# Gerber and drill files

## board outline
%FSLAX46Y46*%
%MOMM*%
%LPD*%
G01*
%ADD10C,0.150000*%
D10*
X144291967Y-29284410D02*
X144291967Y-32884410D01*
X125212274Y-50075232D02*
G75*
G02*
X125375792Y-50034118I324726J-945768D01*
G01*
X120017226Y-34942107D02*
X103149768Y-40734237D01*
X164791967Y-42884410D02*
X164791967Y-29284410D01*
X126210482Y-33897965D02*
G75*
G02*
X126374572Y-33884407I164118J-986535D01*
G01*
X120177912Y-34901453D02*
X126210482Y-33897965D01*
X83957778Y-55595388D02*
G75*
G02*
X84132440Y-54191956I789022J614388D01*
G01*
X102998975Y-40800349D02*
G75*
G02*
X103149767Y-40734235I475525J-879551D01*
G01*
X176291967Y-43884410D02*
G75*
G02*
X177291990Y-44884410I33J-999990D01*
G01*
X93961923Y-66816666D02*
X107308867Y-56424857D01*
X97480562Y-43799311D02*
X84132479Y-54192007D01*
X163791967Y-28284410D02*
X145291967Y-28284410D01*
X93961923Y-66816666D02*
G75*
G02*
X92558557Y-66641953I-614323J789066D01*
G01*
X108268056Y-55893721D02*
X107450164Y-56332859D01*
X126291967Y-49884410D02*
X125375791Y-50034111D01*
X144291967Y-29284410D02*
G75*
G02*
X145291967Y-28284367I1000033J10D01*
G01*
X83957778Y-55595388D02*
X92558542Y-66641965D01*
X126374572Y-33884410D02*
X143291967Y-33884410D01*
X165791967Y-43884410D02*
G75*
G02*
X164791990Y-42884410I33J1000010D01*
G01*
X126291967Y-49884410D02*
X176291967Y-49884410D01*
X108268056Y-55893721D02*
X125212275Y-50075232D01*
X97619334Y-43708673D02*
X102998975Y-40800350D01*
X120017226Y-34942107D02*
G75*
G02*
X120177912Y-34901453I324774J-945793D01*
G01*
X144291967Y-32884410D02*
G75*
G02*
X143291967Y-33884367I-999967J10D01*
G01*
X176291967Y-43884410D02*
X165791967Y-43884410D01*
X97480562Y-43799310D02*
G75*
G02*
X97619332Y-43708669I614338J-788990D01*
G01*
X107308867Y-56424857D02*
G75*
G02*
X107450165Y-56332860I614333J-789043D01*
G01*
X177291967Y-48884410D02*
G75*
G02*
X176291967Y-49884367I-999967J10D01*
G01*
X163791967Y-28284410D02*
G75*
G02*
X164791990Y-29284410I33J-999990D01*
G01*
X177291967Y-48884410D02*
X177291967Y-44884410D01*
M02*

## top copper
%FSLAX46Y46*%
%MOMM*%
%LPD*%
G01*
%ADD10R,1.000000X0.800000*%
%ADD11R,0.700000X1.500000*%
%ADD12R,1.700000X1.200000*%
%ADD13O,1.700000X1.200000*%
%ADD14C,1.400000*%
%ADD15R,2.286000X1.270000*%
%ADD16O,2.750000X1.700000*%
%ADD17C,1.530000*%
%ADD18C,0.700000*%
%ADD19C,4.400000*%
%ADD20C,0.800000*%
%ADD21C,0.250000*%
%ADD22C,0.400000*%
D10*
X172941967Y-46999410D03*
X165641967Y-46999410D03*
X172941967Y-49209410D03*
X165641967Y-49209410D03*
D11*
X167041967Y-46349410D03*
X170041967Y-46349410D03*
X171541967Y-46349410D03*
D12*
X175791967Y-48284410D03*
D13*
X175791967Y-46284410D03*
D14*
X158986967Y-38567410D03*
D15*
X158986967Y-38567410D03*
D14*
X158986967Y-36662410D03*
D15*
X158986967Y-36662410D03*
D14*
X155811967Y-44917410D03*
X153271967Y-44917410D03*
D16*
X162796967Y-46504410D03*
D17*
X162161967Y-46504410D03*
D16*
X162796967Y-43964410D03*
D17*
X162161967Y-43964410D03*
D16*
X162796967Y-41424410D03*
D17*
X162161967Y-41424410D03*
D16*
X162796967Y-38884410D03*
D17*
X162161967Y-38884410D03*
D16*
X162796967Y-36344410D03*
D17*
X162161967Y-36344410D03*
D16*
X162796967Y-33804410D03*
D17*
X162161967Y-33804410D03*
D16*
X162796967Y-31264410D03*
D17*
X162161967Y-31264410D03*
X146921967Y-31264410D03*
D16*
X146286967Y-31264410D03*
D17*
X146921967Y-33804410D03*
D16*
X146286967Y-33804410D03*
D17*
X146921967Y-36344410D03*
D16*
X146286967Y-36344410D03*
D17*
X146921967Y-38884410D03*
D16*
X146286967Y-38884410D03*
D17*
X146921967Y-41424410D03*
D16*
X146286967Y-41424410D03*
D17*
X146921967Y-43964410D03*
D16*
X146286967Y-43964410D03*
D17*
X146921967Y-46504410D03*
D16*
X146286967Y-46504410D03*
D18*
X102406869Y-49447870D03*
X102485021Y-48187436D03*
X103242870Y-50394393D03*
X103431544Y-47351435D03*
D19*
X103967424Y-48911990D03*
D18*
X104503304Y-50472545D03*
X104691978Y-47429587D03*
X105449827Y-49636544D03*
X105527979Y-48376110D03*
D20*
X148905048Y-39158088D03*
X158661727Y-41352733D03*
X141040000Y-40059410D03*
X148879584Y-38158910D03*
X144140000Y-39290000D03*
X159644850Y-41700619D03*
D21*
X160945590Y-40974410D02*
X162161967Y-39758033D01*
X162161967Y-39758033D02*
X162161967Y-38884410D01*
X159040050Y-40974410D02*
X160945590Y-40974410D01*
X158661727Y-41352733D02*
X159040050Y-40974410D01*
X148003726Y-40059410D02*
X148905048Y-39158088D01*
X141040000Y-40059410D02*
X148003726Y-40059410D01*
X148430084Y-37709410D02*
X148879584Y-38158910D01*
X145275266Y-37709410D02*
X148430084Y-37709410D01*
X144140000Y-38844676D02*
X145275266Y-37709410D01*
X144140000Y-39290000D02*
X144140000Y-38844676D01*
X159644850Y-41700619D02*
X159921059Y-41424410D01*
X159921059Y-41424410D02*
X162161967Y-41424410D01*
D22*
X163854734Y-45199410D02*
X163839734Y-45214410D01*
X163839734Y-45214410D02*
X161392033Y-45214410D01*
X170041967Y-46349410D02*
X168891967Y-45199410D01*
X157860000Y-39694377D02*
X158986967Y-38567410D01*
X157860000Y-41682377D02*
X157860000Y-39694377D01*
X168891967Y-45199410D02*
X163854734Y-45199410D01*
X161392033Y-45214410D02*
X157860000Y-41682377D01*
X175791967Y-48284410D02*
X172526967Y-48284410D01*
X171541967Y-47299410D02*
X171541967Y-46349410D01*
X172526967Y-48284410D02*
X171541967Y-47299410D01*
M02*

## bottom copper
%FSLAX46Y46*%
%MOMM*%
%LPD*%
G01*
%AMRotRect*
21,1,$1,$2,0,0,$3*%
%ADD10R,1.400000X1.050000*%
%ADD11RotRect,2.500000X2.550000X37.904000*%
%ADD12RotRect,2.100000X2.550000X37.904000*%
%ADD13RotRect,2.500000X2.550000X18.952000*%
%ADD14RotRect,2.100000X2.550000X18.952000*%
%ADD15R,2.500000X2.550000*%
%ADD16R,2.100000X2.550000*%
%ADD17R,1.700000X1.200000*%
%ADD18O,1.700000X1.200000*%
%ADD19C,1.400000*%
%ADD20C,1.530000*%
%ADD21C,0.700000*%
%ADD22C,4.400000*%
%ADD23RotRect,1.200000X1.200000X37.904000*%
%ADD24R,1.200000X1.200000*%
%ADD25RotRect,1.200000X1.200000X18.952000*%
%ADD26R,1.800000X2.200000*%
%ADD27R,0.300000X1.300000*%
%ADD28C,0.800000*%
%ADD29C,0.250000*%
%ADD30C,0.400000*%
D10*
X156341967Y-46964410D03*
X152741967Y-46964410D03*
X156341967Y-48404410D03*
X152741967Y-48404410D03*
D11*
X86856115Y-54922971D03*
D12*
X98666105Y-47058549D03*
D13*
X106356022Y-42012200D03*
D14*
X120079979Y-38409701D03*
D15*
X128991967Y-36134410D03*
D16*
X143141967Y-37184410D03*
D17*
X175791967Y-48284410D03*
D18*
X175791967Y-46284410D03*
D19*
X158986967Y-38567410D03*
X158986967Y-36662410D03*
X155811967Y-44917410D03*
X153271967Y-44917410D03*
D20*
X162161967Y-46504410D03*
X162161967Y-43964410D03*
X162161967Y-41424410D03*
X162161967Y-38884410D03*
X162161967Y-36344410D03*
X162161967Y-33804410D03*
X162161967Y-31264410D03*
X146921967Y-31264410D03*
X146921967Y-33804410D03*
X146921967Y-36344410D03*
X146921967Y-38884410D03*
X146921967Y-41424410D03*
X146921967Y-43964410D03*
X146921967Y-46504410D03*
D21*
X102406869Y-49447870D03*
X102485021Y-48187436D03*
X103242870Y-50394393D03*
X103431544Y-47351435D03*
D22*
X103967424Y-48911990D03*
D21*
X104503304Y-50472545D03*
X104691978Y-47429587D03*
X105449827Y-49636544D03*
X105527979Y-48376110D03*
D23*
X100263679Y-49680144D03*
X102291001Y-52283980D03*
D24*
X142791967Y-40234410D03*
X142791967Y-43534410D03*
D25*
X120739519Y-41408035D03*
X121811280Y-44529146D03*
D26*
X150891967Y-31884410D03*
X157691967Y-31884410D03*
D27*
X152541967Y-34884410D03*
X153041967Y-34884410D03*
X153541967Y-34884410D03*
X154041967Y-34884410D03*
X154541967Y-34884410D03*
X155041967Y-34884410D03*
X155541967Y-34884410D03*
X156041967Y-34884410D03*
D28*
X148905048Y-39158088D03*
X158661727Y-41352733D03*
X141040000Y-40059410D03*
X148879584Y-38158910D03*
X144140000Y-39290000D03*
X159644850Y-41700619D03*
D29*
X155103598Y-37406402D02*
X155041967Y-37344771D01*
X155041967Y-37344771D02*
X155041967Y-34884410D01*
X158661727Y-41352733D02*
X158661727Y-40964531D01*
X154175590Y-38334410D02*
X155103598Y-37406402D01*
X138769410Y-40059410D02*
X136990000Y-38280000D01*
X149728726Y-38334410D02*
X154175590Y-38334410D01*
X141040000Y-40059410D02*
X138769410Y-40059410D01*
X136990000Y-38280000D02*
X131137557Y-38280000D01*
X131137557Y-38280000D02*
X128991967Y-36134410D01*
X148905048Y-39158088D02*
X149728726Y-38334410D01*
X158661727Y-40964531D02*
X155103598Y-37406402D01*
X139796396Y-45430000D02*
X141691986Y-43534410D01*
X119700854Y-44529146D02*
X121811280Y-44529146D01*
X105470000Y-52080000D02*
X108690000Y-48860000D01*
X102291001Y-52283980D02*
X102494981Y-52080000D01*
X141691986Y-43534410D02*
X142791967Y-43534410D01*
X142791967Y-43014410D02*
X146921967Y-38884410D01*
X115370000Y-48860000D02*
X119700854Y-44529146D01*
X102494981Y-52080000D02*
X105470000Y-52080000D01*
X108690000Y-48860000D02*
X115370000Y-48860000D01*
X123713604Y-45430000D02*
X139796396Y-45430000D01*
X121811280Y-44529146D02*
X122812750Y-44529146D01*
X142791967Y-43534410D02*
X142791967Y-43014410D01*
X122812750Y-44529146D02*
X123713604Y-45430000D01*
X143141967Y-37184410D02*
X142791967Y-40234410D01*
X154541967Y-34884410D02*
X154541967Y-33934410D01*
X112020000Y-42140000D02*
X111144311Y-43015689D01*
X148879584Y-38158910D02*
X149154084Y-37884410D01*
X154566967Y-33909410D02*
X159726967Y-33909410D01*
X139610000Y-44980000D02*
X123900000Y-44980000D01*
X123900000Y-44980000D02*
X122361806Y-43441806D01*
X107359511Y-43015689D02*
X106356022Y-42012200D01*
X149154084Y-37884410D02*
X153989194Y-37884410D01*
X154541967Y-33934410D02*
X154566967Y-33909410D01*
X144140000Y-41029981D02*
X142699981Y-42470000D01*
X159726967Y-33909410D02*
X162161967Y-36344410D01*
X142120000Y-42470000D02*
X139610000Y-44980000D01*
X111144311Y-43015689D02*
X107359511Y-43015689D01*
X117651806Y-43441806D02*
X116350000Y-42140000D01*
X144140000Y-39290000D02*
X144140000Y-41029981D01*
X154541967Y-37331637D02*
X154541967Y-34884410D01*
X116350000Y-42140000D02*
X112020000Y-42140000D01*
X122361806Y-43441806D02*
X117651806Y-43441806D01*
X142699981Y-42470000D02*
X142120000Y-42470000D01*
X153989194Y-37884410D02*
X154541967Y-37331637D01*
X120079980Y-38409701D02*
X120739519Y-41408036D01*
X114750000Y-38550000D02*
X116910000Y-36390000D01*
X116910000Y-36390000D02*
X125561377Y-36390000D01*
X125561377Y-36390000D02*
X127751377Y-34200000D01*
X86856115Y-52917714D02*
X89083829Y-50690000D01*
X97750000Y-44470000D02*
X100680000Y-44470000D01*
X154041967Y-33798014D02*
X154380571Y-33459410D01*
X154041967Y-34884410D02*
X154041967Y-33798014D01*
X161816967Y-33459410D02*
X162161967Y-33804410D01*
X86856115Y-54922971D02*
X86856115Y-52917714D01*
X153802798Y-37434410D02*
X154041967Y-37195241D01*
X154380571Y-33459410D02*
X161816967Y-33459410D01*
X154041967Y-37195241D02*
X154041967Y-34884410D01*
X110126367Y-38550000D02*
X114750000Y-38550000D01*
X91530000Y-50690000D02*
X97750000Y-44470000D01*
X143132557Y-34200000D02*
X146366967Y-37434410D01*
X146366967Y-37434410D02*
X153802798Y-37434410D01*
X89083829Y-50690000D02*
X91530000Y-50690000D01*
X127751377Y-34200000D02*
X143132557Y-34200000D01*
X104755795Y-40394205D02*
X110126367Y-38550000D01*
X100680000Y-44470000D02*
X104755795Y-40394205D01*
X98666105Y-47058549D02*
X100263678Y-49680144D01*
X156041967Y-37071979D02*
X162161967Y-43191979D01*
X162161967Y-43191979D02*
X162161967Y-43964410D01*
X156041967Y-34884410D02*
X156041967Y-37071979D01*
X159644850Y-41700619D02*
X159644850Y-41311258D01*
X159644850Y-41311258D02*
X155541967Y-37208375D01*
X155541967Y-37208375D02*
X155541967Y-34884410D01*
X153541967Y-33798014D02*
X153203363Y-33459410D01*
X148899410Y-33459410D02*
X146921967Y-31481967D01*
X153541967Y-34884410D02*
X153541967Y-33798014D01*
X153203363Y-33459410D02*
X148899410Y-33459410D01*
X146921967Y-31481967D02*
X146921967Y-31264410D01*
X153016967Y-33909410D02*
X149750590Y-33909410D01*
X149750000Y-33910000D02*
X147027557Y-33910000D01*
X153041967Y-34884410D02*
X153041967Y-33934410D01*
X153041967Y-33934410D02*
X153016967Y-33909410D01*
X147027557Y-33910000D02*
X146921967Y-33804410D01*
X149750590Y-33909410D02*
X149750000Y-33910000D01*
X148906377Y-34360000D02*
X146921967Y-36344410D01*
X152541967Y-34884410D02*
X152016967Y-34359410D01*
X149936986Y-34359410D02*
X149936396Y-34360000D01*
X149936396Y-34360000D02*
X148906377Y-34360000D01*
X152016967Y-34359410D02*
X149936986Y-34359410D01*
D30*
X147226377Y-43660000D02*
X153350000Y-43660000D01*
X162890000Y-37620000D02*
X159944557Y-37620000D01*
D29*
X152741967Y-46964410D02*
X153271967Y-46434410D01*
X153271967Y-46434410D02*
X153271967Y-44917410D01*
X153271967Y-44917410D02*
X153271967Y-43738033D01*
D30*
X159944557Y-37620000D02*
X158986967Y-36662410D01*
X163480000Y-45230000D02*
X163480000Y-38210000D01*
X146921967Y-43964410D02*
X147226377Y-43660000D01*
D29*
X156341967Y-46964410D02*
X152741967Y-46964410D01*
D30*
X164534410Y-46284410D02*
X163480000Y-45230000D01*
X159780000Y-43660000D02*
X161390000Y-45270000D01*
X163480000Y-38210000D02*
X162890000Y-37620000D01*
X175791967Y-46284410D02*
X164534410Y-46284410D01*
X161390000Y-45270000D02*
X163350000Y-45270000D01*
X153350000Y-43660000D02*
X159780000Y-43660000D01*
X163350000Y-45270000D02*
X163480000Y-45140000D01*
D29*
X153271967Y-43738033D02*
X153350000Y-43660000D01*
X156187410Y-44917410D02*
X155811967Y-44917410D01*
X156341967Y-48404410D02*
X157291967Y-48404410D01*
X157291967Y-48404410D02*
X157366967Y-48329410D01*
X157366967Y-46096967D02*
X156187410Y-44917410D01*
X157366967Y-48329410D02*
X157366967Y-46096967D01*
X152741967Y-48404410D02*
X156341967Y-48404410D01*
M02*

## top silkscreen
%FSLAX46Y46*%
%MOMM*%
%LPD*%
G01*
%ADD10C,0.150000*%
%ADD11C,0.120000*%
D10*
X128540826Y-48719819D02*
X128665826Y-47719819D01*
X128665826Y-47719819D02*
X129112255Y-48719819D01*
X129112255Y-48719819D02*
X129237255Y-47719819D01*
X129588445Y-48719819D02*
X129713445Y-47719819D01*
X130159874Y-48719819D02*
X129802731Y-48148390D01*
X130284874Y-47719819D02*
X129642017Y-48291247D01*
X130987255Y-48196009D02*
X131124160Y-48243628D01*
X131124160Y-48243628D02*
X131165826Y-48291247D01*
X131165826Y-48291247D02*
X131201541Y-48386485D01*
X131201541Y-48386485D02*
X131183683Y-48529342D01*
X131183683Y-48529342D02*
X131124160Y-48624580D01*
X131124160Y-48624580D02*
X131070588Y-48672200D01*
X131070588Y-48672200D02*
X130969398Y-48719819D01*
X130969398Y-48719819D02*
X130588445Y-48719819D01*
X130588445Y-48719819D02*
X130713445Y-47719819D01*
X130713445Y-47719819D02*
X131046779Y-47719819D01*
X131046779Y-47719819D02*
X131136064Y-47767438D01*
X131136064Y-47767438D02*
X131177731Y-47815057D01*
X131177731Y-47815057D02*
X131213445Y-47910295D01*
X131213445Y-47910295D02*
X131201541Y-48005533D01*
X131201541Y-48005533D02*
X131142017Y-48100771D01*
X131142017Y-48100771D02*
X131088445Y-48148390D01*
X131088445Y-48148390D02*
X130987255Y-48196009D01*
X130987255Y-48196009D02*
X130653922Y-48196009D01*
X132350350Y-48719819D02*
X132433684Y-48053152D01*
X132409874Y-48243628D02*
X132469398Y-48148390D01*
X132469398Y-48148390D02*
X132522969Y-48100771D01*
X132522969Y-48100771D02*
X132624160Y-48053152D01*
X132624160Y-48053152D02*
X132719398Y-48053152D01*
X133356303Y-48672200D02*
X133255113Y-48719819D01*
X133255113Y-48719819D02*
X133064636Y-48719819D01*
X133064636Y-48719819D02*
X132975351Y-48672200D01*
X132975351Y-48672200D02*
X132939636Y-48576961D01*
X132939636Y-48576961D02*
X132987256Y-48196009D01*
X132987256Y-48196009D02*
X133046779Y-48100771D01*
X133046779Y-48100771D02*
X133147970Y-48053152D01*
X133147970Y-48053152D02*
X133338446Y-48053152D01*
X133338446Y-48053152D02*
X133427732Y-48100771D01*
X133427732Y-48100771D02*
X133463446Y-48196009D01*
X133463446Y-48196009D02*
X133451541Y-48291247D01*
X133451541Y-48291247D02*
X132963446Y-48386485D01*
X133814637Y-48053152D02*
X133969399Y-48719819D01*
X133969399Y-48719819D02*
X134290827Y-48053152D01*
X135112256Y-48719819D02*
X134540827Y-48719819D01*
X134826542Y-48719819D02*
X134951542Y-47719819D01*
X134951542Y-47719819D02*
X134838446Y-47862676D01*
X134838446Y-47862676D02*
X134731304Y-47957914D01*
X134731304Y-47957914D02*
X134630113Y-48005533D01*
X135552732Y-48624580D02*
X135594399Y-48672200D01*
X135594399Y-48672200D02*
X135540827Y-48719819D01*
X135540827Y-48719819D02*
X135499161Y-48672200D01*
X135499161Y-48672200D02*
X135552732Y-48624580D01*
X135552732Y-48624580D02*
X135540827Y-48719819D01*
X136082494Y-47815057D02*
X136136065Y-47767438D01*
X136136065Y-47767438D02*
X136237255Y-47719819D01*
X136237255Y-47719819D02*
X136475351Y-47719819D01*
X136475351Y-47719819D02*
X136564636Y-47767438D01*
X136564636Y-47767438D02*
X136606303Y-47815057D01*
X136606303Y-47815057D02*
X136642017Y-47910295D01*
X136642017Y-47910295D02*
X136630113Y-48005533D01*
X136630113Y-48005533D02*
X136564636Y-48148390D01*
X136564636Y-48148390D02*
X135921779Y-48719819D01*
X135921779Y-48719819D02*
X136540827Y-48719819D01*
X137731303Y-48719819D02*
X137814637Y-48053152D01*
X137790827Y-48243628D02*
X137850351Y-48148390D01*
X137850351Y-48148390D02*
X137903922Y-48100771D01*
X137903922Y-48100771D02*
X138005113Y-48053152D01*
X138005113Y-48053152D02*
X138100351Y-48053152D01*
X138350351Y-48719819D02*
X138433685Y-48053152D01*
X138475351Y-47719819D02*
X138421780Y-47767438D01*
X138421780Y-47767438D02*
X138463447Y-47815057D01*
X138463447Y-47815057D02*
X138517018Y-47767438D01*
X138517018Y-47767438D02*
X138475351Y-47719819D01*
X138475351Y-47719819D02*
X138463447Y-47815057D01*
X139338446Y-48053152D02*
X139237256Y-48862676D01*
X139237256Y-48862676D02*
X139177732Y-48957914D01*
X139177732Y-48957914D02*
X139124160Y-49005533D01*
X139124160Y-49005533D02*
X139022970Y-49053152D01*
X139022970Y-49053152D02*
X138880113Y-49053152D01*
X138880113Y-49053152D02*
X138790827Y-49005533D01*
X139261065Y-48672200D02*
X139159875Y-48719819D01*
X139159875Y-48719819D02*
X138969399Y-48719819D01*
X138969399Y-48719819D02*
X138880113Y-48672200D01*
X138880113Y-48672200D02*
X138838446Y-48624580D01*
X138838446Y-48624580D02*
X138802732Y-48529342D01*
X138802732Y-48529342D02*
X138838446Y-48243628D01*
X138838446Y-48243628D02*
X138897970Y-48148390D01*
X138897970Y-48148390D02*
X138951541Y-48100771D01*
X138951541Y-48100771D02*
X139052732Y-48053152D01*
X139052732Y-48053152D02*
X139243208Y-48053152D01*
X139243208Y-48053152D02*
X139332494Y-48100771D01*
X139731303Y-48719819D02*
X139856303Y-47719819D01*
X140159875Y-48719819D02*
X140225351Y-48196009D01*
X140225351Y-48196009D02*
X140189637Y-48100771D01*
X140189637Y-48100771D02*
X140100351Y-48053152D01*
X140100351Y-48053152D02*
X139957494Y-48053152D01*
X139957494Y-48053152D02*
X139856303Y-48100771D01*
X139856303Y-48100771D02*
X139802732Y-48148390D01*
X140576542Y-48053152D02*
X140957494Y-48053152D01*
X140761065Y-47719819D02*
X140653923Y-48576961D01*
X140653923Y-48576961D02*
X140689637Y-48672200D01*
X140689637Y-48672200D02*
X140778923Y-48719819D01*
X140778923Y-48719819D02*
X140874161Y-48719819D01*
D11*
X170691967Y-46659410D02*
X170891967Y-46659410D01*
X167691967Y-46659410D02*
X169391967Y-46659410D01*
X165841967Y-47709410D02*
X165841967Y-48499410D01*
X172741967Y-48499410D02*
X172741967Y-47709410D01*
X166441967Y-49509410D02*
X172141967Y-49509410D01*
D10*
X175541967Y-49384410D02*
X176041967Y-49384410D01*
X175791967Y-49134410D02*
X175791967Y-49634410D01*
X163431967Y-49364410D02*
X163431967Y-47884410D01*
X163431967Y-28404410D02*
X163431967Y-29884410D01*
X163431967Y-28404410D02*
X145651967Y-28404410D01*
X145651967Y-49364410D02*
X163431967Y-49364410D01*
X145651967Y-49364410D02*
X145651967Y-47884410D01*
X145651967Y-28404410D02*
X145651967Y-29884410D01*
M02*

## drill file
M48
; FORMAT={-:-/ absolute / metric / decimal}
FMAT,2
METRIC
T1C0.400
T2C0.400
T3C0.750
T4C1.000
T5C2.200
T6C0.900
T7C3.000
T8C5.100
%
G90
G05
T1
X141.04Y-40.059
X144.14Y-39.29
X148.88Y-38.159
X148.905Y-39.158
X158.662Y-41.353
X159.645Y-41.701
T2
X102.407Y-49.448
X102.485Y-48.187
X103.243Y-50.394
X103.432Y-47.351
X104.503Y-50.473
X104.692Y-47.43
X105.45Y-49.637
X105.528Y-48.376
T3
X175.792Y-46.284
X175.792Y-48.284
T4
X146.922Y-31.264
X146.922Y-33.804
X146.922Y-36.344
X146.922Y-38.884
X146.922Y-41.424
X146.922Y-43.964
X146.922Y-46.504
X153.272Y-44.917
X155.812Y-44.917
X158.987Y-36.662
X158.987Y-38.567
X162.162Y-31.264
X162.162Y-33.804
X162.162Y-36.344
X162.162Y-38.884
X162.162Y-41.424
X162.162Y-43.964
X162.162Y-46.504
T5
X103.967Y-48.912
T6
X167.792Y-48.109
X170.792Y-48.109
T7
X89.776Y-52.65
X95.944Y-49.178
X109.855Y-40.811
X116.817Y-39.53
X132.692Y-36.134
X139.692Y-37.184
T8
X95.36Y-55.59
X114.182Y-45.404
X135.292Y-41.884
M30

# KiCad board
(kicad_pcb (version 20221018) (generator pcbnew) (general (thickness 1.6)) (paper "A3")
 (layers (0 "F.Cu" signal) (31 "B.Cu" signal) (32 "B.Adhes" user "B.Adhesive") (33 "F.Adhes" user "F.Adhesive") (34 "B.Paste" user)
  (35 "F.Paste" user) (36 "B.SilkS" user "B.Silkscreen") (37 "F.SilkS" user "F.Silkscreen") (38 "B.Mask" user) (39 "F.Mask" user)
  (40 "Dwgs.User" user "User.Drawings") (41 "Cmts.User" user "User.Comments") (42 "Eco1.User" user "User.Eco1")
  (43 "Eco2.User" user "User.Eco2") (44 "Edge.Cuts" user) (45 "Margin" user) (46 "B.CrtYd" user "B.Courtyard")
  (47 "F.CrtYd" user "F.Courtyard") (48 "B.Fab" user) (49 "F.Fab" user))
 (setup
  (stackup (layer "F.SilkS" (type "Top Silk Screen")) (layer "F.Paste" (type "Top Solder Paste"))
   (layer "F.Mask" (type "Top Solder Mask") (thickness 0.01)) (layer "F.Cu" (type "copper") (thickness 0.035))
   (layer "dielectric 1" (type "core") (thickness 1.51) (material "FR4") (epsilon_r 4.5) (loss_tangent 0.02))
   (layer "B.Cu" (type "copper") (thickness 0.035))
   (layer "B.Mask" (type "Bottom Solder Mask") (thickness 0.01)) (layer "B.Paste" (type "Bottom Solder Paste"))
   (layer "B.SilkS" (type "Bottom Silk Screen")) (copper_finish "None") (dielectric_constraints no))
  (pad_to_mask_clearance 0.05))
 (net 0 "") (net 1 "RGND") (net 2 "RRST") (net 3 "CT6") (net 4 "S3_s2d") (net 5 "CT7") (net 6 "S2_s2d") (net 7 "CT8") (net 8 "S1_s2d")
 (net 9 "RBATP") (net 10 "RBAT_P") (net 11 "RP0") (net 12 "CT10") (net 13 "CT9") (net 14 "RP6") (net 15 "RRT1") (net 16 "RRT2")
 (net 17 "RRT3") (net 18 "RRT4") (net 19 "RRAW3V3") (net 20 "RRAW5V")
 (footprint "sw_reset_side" (layer "F.Cu") (at 154.541967 47.68441 -90)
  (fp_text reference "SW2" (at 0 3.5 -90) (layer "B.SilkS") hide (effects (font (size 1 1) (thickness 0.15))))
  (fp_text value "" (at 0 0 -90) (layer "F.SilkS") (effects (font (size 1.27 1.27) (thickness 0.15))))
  (pad "1" smd rect (at -0.72 -1.8 180) (size 1.4 1.05) (layers "B.Cu" "B.Paste" "B.Mask") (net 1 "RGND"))
  (pad "1" smd rect (at -0.72 1.8 180) (size 1.4 1.05) (layers "B.Cu" "B.Paste" "B.Mask") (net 1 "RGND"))
  (pad "2" smd rect (at 0.72 -1.8 180) (size 1.4 1.05) (layers "B.Cu" "B.Paste" "B.Mask") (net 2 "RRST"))
  (pad "2" smd rect (at 0.72 1.8 180) (size 1.4 1.05) (layers "B.Cu" "B.Paste" "B.Mask") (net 2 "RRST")))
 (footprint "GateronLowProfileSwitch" (layer "F.Cu") (at 95.359531 55.589614 37.904)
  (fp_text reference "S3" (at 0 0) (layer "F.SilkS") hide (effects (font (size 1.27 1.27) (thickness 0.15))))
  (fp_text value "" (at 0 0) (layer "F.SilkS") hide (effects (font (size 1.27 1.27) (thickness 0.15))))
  (pad "" np_thru_hole circle (at -2.6 -5.75) (size 3 3) (drill 3) (layers "*.Cu" "*.Mask"))
  (pad "" np_thru_hole circle (at 0 0) (size 5.1 5.1) (drill 5.1) (layers "*.Cu" "*.Mask"))
  (pad "" np_thru_hole circle (at 4.4 -4.7) (size 3 3) (drill 3) (layers "*.Cu" "*.Mask"))
  (pad "1" smd rect (at -6.3 -5.75 37.904) (size 2.5 2.55) (layers "B.Cu" "B.Paste" "B.Mask") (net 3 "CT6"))
  (pad "2" smd rect (at 7.85 -4.7 37.904) (size 2.1 2.55) (layers "B.Cu" "B.Paste" "B.Mask") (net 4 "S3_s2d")))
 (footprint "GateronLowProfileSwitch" (layer "F.Cu") (at 114.181967 45.40441 18.952)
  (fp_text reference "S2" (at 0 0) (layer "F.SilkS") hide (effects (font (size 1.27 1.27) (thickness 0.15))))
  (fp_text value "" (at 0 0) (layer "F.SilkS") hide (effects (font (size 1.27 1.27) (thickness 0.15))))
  (pad "" np_thru_hole circle (at -2.6 -5.75) (size 3 3) (drill 3) (layers "*.Cu" "*.Mask"))
  (pad "" np_thru_hole circle (at 0 0) (size 5.1 5.1) (drill 5.1) (layers "*.Cu" "*.Mask"))
  (pad "" np_thru_hole circle (at 4.4 -4.7) (size 3 3) (drill 3) (layers "*.Cu" "*.Mask"))
  (pad "1" smd rect (at -6.3 -5.75 18.952) (size 2.5 2.55) (layers "B.Cu" "B.Paste" "B.Mask") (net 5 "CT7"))
  (pad "2" smd rect (at 7.85 -4.7 18.952) (size 2.1 2.55) (layers "B.Cu" "B.Paste" "B.Mask") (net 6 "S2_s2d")))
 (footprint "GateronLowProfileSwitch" (layer "F.Cu") (at 135.291967 41.88441)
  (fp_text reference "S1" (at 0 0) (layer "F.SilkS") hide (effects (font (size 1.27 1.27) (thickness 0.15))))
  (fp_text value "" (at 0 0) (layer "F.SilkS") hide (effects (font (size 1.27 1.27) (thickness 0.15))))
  (pad "" np_thru_hole circle (at -2.6 -5.75) (size 3 3) (drill 3) (layers "*.Cu" "*.Mask"))
  (pad "" np_thru_hole circle (at 0 0) (size 5.1 5.1) (drill 5.1) (layers "*.Cu" "*.Mask"))
  (pad "" np_thru_hole circle (at 4.4 -4.7) (size 3 3) (drill 3) (layers "*.Cu" "*.Mask"))
  (pad "1" smd rect (at -6.3 -5.75) (size 2.5 2.55) (layers "B.Cu" "B.Paste" "B.Mask") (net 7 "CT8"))
  (pad "2" smd rect (at 7.85 -4.7) (size 2.1 2.55) (layers "B.Cu" "B.Paste" "B.Mask") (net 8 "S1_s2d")))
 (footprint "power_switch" (layer "F.Cu") (at 169.291967 48.08441 -90)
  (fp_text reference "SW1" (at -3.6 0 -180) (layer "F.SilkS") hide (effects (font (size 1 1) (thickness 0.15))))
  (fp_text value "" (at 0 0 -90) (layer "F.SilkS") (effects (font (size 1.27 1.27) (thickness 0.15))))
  (fp_line (start -1.425 -1.4) (end -1.425 -1.6) (stroke (width 0.12) (type solid)) (layer "F.SilkS"))
  (fp_line (start -1.425 1.6) (end -1.425 -0.1) (stroke (width 0.12) (type solid)) (layer "F.SilkS"))
  (fp_line (start -0.375 3.45) (end 0.415 3.45) (stroke (width 0.12) (type solid)) (layer "F.SilkS"))
  (fp_line (start 0.415 -3.45) (end -0.375 -3.45) (stroke (width 0.12) (type solid)) (layer "F.SilkS"))
  (fp_line (start 1.425 2.85) (end 1.425 -2.85) (stroke (width 0.12) (type solid)) (layer "F.SilkS"))
  (pad "" smd rect (at -1.085 -3.65) (size 1 0.8) (layers "F.Cu" "F.Paste" "F.Mask"))
  (pad "" smd rect (at -1.085 3.65) (size 1 0.8) (layers "F.Cu" "F.Paste" "F.Mask"))
  (pad "" np_thru_hole circle (at 0.025 -1.5) (size 0.9 0.9) (drill 0.9) (layers "*.Cu" "*.Mask"))
  (pad "" np_thru_hole circle (at 0.025 1.5) (size 0.9 0.9) (drill 0.9) (layers "*.Cu" "*.Mask"))
  (pad "" smd rect (at 1.125 -3.65) (size 1 0.8) (layers "F.Cu" "F.Paste" "F.Mask"))
  (pad "" smd rect (at 1.125 3.65) (size 1 0.8) (layers "F.Cu" "F.Paste" "F.Mask"))
  (pad "1" smd rect (at -1.735 2.25) (size 0.7 1.5) (layers "F.Cu" "F.Paste" "F.Mask"))
  (pad "2" smd rect (at -1.735 -0.75) (size 0.7 1.5) (layers "F.Cu" "F.Paste" "F.Mask") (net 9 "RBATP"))
  (pad "3" smd rect (at -1.735 -2.25) (size 0.7 1.5) (layers "F.Cu" "F.Paste" "F.Mask") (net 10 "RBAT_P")))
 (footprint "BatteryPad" (layer "F.Cu") (at 175.791967 47.28441 90)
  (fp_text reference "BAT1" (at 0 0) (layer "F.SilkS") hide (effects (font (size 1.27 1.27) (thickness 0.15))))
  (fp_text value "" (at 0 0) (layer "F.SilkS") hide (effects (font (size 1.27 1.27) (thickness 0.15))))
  (fp_line (start -2.1 -0.25) (end -2.1 0.25) (stroke (width 0.15) (type solid)) (layer "F.SilkS"))
  (fp_line (start -1.85 0) (end -2.35 0) (stroke (width 0.15) (type solid)) (layer "F.SilkS"))
  (pad "1" thru_hole rect (at -1 0 90) (size 1.2 1.7) (drill 0.75) (layers "*.Cu" "*.Mask") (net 10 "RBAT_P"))
  (pad "2" thru_hole oval (at 1 0 90) (size 1.2 1.7) (drill 0.75) (layers "*.Cu" "*.Mask") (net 1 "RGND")))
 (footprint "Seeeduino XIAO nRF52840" (layer "F.Cu") (at 154.541967 38.88441 180)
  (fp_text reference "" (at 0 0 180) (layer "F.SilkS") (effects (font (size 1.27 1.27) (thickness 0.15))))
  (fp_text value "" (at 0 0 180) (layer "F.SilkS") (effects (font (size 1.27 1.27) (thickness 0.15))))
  (fp_line (start -8.89 -10.48) (end -8.89 -9) (stroke (width 0.15) (type solid)) (layer "F.SilkS"))
  (fp_line (start -8.89 10.48) (end -8.89 9) (stroke (width 0.15) (type solid)) (layer "F.SilkS"))
  (fp_line (start -8.89 10.48) (end 8.89 10.48) (stroke (width 0.15) (type solid)) (layer "F.SilkS"))
  (fp_line (start 8.89 -10.48) (end -8.89 -10.48) (stroke (width 0.15) (type solid)) (layer "F.SilkS"))
  (fp_line (start 8.89 -10.48) (end 8.89 -9) (stroke (width 0.15) (type solid)) (layer "F.SilkS"))
  (fp_line (start 8.89 10.48) (end 8.89 9) (stroke (width 0.15) (type solid)) (layer "F.SilkS"))
  (pad "" thru_hole circle (at -4.445 0.317) (size 1.4 1.4) (drill 1) (layers "*.Cu" "*.Mask") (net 9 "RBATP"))
  (pad "" smd rect (at -4.445 0.317 180) (size 2.286 1.27) (layers "F.Cu" "F.Paste" "F.Mask") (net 9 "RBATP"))
  (pad "" thru_hole circle (at -4.445 2.222) (size 1.4 1.4) (drill 1) (layers "*.Cu" "*.Mask") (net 1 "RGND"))
  (pad "" smd rect (at -4.445 2.222 180) (size 2.286 1.27) (layers "F.Cu" "F.Paste" "F.Mask") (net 1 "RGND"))
  (pad "" thru_hole circle (at -1.27 -6.033) (size 1.4 1.4) (drill 1) (layers "*.Cu" "*.Mask") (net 2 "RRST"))
  (pad "" thru_hole circle (at 1.27 -6.033) (size 1.4 1.4) (drill 1) (layers "*.Cu" "*.Mask") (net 1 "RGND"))
  (pad "1" smd oval (at -8.255 -7.62 180) (size 2.75 1.7) (layers "F.Cu" "F.Paste" "F.Mask") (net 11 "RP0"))
  (pad "1" thru_hole circle (at -7.62 -7.62) (size 1.53 1.53) (drill 1) (layers "*.Cu" "*.Mask") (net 11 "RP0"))
  (pad "2" smd oval (at -8.255 -5.08 180) (size 2.75 1.7) (layers "F.Cu" "F.Paste" "F.Mask") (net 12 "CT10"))
  (pad "2" thru_hole circle (at -7.62 -5.08) (size 1.53 1.53) (drill 1) (layers "*.Cu" "*.Mask") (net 12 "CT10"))
  (pad "3" smd oval (at -8.255 -2.54 180) (size 2.75 1.7) (layers "F.Cu" "F.Paste" "F.Mask") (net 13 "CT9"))
  (pad "3" thru_hole circle (at -7.62 -2.54) (size 1.53 1.53) (drill 1) (layers "*.Cu" "*.Mask") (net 13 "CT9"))
  (pad "4" smd oval (at -8.255 0 180) (size 2.75 1.7) (layers "F.Cu" "F.Paste" "F.Mask") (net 7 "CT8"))
  (pad "4" thru_hole circle (at -7.62 0) (size 1.53 1.53) (drill 1) (layers "*.Cu" "*.Mask") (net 7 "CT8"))
  (pad "5" smd oval (at -8.255 2.54 180) (size 2.75 1.7) (layers "F.Cu" "F.Paste" "F.Mask") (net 5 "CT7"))
  (pad "5" thru_hole circle (at -7.62 2.54) (size 1.53 1.53) (drill 1) (layers "*.Cu" "*.Mask") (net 5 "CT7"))
  (pad "6" smd oval (at -8.255 5.08 180) (size 2.75 1.7) (layers "F.Cu" "F.Paste" "F.Mask") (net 3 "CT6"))
  (pad "6" thru_hole circle (at -7.62 5.08) (size 1.53 1.53) (drill 1) (layers "*.Cu" "*.Mask") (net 3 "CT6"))
  (pad "7" smd oval (at -8.255 7.62 180) (size 2.75 1.7) (layers "F.Cu" "F.Paste" "F.Mask") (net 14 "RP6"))
  (pad "7" thru_hole circle (at -7.62 7.62) (size 1.53 1.53) (drill 1) (layers "*.Cu" "*.Mask") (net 14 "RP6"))
  (pad "8" thru_hole circle (at 7.62 7.62) (size 1.53 1.53) (drill 1) (layers "*.Cu" "*.Mask") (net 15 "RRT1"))
  (pad "8" smd oval (at 8.255 7.62 180) (size 2.75 1.7) (layers "F.Cu" "F.Paste" "F.Mask") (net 15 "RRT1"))
  (pad "9" thru_hole circle (at 7.62 5.08) (size 1.53 1.53) (drill 1) (layers "*.Cu" "*.Mask") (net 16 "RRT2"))
  (pad "9" smd oval (at 8.255 5.08 180) (size 2.75 1.7) (layers "F.Cu" "F.Paste" "F.Mask") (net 16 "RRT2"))
  (pad "10" thru_hole circle (at 7.62 2.54) (size 1.53 1.53) (drill 1) (layers "*.Cu" "*.Mask") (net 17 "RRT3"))
  (pad "10" smd oval (at 8.255 2.54 180) (size 2.75 1.7) (layers "F.Cu" "F.Paste" "F.Mask") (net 17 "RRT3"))
  (pad "11" thru_hole circle (at 7.62 0) (size 1.53 1.53) (drill 1) (layers "*.Cu" "*.Mask") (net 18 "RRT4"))
  (pad "11" smd oval (at 8.255 0 180) (size 2.75 1.7) (layers "F.Cu" "F.Paste" "F.Mask") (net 18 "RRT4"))
  (pad "12" thru_hole circle (at 7.62 -2.54) (size 1.53 1.53) (drill 1) (layers "*.Cu" "*.Mask") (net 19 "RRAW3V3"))
  (pad "12" smd oval (at 8.255 -2.54 180) (size 2.75 1.7) (layers "F.Cu" "F.Paste" "F.Mask") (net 19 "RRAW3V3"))
  (pad "13" thru_hole circle (at 7.62 -5.08) (size 1.53 1.53) (drill 1) (layers "*.Cu" "*.Mask") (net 1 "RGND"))
  (pad "13" smd oval (at 8.255 -5.08 180) (size 2.75 1.7) (layers "F.Cu" "F.Paste" "F.Mask") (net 1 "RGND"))
  (pad "14" thru_hole circle (at 7.62 -7.62) (size 1.53 1.53) (drill 1) (layers "*.Cu" "*.Mask") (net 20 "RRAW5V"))
  (pad "14" smd oval (at 8.255 -7.62 180) (size 2.75 1.7) (layers "F.Cu" "F.Paste" "F.Mask") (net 20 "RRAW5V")))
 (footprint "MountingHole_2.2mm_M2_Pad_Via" (layer "F.Cu") (at 103.967424 48.91199 18.952)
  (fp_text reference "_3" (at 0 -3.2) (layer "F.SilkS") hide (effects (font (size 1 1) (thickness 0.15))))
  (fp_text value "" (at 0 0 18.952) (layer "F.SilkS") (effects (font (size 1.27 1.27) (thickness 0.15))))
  (pad "1" thru_hole circle (at -1.65 0) (size 0.7 0.7) (drill 0.4) (layers "*.Cu" "*.Mask"))
  (pad "1" thru_hole circle (at -1.166726 -1.166726) (size 0.7 0.7) (drill 0.4) (layers "*.Cu" "*.Mask"))
  (pad "1" thru_hole circle (at -1.166726 1.166726) (size 0.7 0.7) (drill 0.4) (layers "*.Cu" "*.Mask"))
  (pad "1" thru_hole circle (at 0 -1.65) (size 0.7 0.7) (drill 0.4) (layers "*.Cu" "*.Mask"))
  (pad "1" thru_hole circle (at 0 0) (size 4.4 4.4) (drill 2.2) (layers "*.Cu" "*.Mask"))
  (pad "1" thru_hole circle (at 0 1.65) (size 0.7 0.7) (drill 0.4) (layers "*.Cu" "*.Mask"))
  (pad "1" thru_hole circle (at 1.166726 -1.166726) (size 0.7 0.7) (drill 0.4) (layers "*.Cu" "*.Mask"))
  (pad "1" thru_hole circle (at 1.166726 1.166726) (size 0.7 0.7) (drill 0.4) (layers "*.Cu" "*.Mask"))
  (pad "1" thru_hole circle (at 1.65 0) (size 0.7 0.7) (drill 0.4) (layers "*.Cu" "*.Mask")))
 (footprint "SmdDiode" (layer "B.Cu") (at 95.359531 55.589614 37.904)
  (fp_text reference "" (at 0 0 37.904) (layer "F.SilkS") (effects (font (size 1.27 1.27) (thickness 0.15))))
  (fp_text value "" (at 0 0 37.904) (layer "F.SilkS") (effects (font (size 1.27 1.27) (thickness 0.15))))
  (pad "1" smd rect (at 7.5 -1.65 37.904) (size 1.2 1.2) (layers "B.Cu" "B.Paste" "B.Mask") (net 4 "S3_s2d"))
  (pad "2" smd rect (at 7.5 1.65 37.904) (size 1.2 1.2) (layers "B.Cu" "B.Paste" "B.Mask") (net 18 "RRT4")))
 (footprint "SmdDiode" (layer "B.Cu") (at 135.291967 41.88441)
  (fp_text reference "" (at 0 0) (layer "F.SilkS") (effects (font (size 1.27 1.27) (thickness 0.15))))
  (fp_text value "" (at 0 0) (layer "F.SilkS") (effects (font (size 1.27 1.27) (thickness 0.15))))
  (pad "1" smd rect (at 7.5 -1.65) (size 1.2 1.2) (layers "B.Cu" "B.Paste" "B.Mask") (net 8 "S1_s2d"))
  (pad "2" smd rect (at 7.5 1.65) (size 1.2 1.2) (layers "B.Cu" "B.Paste" "B.Mask") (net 18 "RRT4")))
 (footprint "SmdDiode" (layer "B.Cu") (at 114.181967 45.40441 18.952)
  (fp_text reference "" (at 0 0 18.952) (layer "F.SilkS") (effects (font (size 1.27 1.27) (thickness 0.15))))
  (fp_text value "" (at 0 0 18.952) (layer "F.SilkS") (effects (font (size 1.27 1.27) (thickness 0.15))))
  (pad "1" smd rect (at 7.5 -1.65 18.952) (size 1.2 1.2) (layers "B.Cu" "B.Paste" "B.Mask") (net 6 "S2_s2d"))
  (pad "2" smd rect (at 7.5 1.65 18.952) (size 1.2 1.2) (layers "B.Cu" "B.Paste" "B.Mask") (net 18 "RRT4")))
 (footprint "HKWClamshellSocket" (layer "B.Cu") (at 154.291967 31.88441)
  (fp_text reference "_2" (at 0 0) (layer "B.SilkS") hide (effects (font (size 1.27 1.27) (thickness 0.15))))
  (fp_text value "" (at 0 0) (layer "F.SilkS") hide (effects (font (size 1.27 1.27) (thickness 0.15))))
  (pad "" smd rect (at -3.4 0) (size 1.8 2.2) (layers "B.Cu" "B.Paste" "B.Mask"))
  (pad "" smd rect (at 3.4 0) (size 1.8 2.2) (layers "B.Cu" "B.Paste" "B.Mask"))
  (pad "1" smd rect (at -1.75 3) (size 0.3 1.3) (layers "B.Cu" "B.Paste" "B.Mask") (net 17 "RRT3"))
  (pad "2" smd rect (at -1.25 3) (size 0.3 1.3) (layers "B.Cu" "B.Paste" "B.Mask") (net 16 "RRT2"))
  (pad "3" smd rect (at -0.75 3) (size 0.3 1.3) (layers "B.Cu" "B.Paste" "B.Mask") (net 15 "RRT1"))
  (pad "4" smd rect (at -0.25 3) (size 0.3 1.3) (layers "B.Cu" "B.Paste" "B.Mask") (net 3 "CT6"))
  (pad "5" smd rect (at 0.25 3) (size 0.3 1.3) (layers "B.Cu" "B.Paste" "B.Mask") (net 5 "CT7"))
  (pad "6" smd rect (at 0.75 3) (size 0.3 1.3) (layers "B.Cu" "B.Paste" "B.Mask") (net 7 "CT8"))
  (pad "7" smd rect (at 1.25 3) (size 0.3 1.3) (layers "B.Cu" "B.Paste" "B.Mask") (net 13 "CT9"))
  (pad "8" smd rect (at 1.75 3) (size 0.3 1.3) (layers "B.Cu" "B.Paste" "B.Mask") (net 12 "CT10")))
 (gr_line (start 144.291967 29.28441) (end 144.291967 32.88441) (stroke (width 0.15) (type solid)) (layer "Edge.Cuts"))
 (gr_arc (start 125.212274 50.075232) (mid 125.293164 50.051219) (end 125.375791 50.034111) (stroke (width 0.15) (type solid))
  (layer "Edge.Cuts"))
 (gr_line (start 120.017226 34.942107) (end 103.149768 40.734237) (stroke (width 0.15) (type solid)) (layer "Edge.Cuts"))
 (gr_line (start 164.791967 42.88441) (end 164.791967 29.28441) (stroke (width 0.15) (type solid)) (layer "Edge.Cuts"))
 (gr_arc (start 126.210482 33.897965) (mid 126.292248 33.887805) (end 126.374572 33.88441) (stroke (width 0.15) (type solid))
  (layer "Edge.Cuts"))
 (gr_line (start 120.177912 34.901453) (end 126.210482 33.897965) (stroke (width 0.15) (type solid)) (layer "Edge.Cuts"))
 (gr_arc (start 83.957778 55.595388) (mid 83.754479 54.857516) (end 84.132479 54.192007) (stroke (width 0.15) (type solid))
  (layer "Edge.Cuts"))
 (gr_arc (start 102.998975 40.800349) (mid 103.073008 40.764184) (end 103.149768 40.734237) (stroke (width 0.15) (type solid))
  (layer "Edge.Cuts"))
 (gr_arc (start 176.291967 43.88441) (mid 176.999074 44.177303) (end 177.291967 44.88441) (stroke (width 0.15) (type solid))
  (layer "Edge.Cuts"))
 (gr_line (start 93.961923 66.816666) (end 107.308867 56.424857) (stroke (width 0.15) (type solid)) (layer "Edge.Cuts"))
 (gr_line (start 97.480562 43.799311) (end 84.132479 54.192007) (stroke (width 0.15) (type solid)) (layer "Edge.Cuts"))
 (gr_line (start 163.791967 28.28441) (end 145.291967 28.28441) (stroke (width 0.15) (type solid)) (layer "Edge.Cuts"))
 (gr_arc (start 93.961923 66.816666) (mid 93.224051 67.019965) (end 92.558542 66.641965) (stroke (width 0.15) (type solid))
  (layer "Edge.Cuts"))
 (gr_line (start 108.268056 55.893721) (end 107.450164 56.332859) (stroke (width 0.15) (type solid)) (layer "Edge.Cuts"))
 (gr_line (start 126.291967 49.88441) (end 125.375791 50.034111) (stroke (width 0.15) (type solid)) (layer "Edge.Cuts"))
 (gr_arc (start 144.291967 29.28441) (mid 144.58486 28.577303) (end 145.291967 28.28441) (stroke (width 0.15) (type solid))
  (layer "Edge.Cuts"))
 (gr_line (start 83.957778 55.595388) (end 92.558542 66.641965) (stroke (width 0.15) (type solid)) (layer "Edge.Cuts"))
 (gr_line (start 126.374572 33.88441) (end 143.291967 33.88441) (stroke (width 0.15) (type solid)) (layer "Edge.Cuts"))
 (gr_arc (start 165.791967 43.88441) (mid 165.08486 43.591517) (end 164.791967 42.88441) (stroke (width 0.15) (type solid))
  (layer "Edge.Cuts"))
 (gr_line (start 126.291967 49.88441) (end 176.291967 49.88441) (stroke (width 0.15) (type solid)) (layer "Edge.Cuts"))
 (gr_line (start 108.268056 55.893721) (end 125.212275 50.075232) (stroke (width 0.15) (type solid)) (layer "Edge.Cuts"))
 (gr_line (start 97.619334 43.708673) (end 102.998975 40.80035) (stroke (width 0.15) (type solid)) (layer "Edge.Cuts"))
 (gr_arc (start 120.017226 34.942107) (mid 120.096725 34.918445) (end 120.177912 34.901453) (stroke (width 0.15) (type solid))
  (layer "Edge.Cuts"))
 (gr_arc (start 144.291967 32.88441) (mid 143.999074 33.591517) (end 143.291967 33.88441) (stroke (width 0.15) (type solid))
  (layer "Edge.Cuts"))
 (gr_line (start 176.291967 43.88441) (end 165.791967 43.88441) (stroke (width 0.15) (type solid)) (layer "Edge.Cuts"))
 (gr_arc (start 97.480562 43.79931) (mid 97.548067 43.751111) (end 97.619334 43.708673) (stroke (width 0.15) (type solid))
  (layer "Edge.Cuts"))
 (gr_arc (start 107.308867 56.424857) (mid 107.377573 56.375875) (end 107.450164 56.332859) (stroke (width 0.15) (type solid))
  (layer "Edge.Cuts"))
 (gr_arc (start 177.291967 48.88441) (mid 176.999074 49.591517) (end 176.291967 49.88441) (stroke (width 0.15) (type solid))
  (layer "Edge.Cuts"))
 (gr_arc (start 163.791967 28.28441) (mid 164.499074 28.577303) (end 164.791967 29.28441) (stroke (width 0.15) (type solid))
  (layer "Edge.Cuts"))
 (gr_line (start 177.291967 48.88441) (end 177.291967 44.88441) (stroke (width 0.15) (type solid)) (layer "Edge.Cuts"))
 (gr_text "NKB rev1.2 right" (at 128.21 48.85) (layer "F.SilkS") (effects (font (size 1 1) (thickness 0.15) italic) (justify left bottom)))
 (segment (start 160.94559 40.97441) (end 162.161967 39.758033) (width 0.25) (layer "F.Cu") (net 7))
 (segment (start 162.161967 39.758033) (end 162.161967 38.88441) (width 0.25) (layer "F.Cu") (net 7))
 (segment (start 159.04005 40.97441) (end 160.94559 40.97441) (width 0.25) (layer "F.Cu") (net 7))
 (segment (start 158.661727 41.352733) (end 159.04005 40.97441) (width 0.25) (layer "F.Cu") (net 7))
 (segment (start 148.003726 40.05941) (end 148.905048 39.158088) (width 0.25) (layer "F.Cu") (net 7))
 (segment (start 141.04 40.05941) (end 148.003726 40.05941) (width 0.25) (layer "F.Cu") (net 7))
 (via (at 148.905048 39.158088) (size 0.8) (drill 0.4) (layers "F.Cu" "B.Cu") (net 7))
 (via (at 158.661727 41.352733) (size 0.8) (drill 0.4) (layers "F.Cu" "B.Cu") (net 7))
 (via (at 141.04 40.05941) (size 0.8) (drill 0.4) (layers "F.Cu" "B.Cu") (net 7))
 (segment (start 155.103598 37.406402) (end 155.041967 37.344771) (width 0.25) (layer "B.Cu") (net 7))
 (segment (start 155.041967 37.344771) (end 155.041967 34.88441) (width 0.25) (layer "B.Cu") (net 7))
 (segment (start 158.661727 41.352733) (end 158.661727 40.964531) (width 0.25) (layer "B.Cu") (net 7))
 (segment (start 154.17559 38.33441) (end 155.103598 37.406402) (width 0.25) (layer "B.Cu") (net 7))
 (segment (start 138.76941 40.05941) (end 136.99 38.28) (width 0.25) (layer "B.Cu") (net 7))
 (segment (start 149.728726 38.33441) (end 154.17559 38.33441) (width 0.25) (layer "B.Cu") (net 7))
 (segment (start 141.04 40.05941) (end 138.76941 40.05941) (width 0.25) (layer "B.Cu") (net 7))
 (segment (start 136.99 38.28) (end 131.137557 38.28) (width 0.25) (layer "B.Cu") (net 7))
 (segment (start 131.137557 38.28) (end 128.991967 36.13441) (width 0.25) (layer "B.Cu") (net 7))
 (segment (start 148.905048 39.158088) (end 149.728726 38.33441) (width 0.25) (layer "B.Cu") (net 7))
 (segment (start 158.661727 40.964531) (end 155.103598 37.406402) (width 0.25) (layer "B.Cu") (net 7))
 (segment (start 139.796396 45.43) (end 141.691986 43.53441) (width 0.25) (layer "B.Cu") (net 18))
 (segment (start 119.700854 44.529146) (end 121.81128 44.529146) (width 0.25) (layer "B.Cu") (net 18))
 (segment (start 105.47 52.08) (end 108.69 48.86) (width 0.25) (layer "B.Cu") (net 18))
 (segment (start 102.291001 52.28398) (end 102.494981 52.08) (width 0.25) (layer "B.Cu") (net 18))
 (segment (start 141.691986 43.53441) (end 142.791967 43.53441) (width 0.25) (layer "B.Cu") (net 18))
 (segment (start 142.791967 43.01441) (end 146.921967 38.88441) (width 0.25) (layer "B.Cu") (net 18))
 (segment (start 115.37 48.86) (end 119.700854 44.529146) (width 0.25) (layer "B.Cu") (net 18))
 (segment (start 102.494981 52.08) (end 105.47 52.08) (width 0.25) (layer "B.Cu") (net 18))
 (segment (start 108.69 48.86) (end 115.37 48.86) (width 0.25) (layer "B.Cu") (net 18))
 (segment (start 123.713604 45.43) (end 139.796396 45.43) (width 0.25) (layer "B.Cu") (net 18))
 (segment (start 121.81128 44.529146) (end 122.81275 44.529146) (width 0.25) (layer "B.Cu") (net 18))
 (segment (start 142.791967 43.53441) (end 142.791967 43.01441) (width 0.25) (layer "B.Cu") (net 18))
 (segment (start 122.81275 44.529146) (end 123.713604 45.43) (width 0.25) (layer "B.Cu") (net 18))
 (segment (start 143.141967 37.18441) (end 142.791967 40.23441) (width 0.25) (layer "B.Cu") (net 8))
 (segment (start 148.430084 37.70941) (end 148.879584 38.15891) (width 0.25) (layer "F.Cu") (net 5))
 (segment (start 145.275266 37.70941) (end 148.430084 37.70941) (width 0.25) (layer "F.Cu") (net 5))
 (segment (start 144.14 38.844676) (end 145.275266 37.70941) (width 0.25) (layer "F.Cu") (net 5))
 (segment (start 144.14 39.29) (end 144.14 38.844676) (width 0.25) (layer "F.Cu") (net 5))
 (via (at 148.879584 38.15891) (size 0.8) (drill 0.4) (layers "F.Cu" "B.Cu") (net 5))
 (via (at 144.14 39.29) (size 0.8) (drill 0.4) (layers "F.Cu" "B.Cu") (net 5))
 (segment (start 154.541967 34.88441) (end 154.541967 33.93441) (width 0.25) (layer "B.Cu") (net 5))
 (segment (start 112.02 42.14) (end 111.144311 43.015689) (width 0.25) (layer "B.Cu") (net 5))
 (segment (start 148.879584 38.15891) (end 149.154084 37.88441) (width 0.25) (layer "B.Cu") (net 5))
 (segment (start 154.566967 33.90941) (end 159.726967 33.90941) (width 0.25) (layer "B.Cu") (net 5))
 (segment (start 139.61 44.98) (end 123.9 44.98) (width 0.25) (layer "B.Cu") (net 5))
 (segment (start 123.9 44.98) (end 122.361806 43.441806) (width 0.25) (layer "B.Cu") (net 5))
 (segment (start 107.359511 43.015689) (end 106.356022 42.0122) (width 0.25) (layer "B.Cu") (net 5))
 (segment (start 149.154084 37.88441) (end 153.989194 37.88441) (width 0.25) (layer "B.Cu") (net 5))
 (segment (start 154.541967 33.93441) (end 154.566967 33.90941) (width 0.25) (layer "B.Cu") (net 5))
 (segment (start 144.14 41.029981) (end 142.699981 42.47) (width 0.25) (layer "B.Cu") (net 5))
 (segment (start 159.726967 33.90941) (end 162.161967 36.34441) (width 0.25) (layer "B.Cu") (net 5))
 (segment (start 142.12 42.47) (end 139.61 44.98) (width 0.25) (layer "B.Cu") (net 5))
 (segment (start 111.144311 43.015689) (end 107.359511 43.015689) (width 0.25) (layer "B.Cu") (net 5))
 (segment (start 117.651806 43.441806) (end 116.35 42.14) (width 0.25) (layer "B.Cu") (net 5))
 (segment (start 144.14 39.29) (end 144.14 41.029981) (width 0.25) (layer "B.Cu") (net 5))
 (segment (start 154.541967 37.331637) (end 154.541967 34.88441) (width 0.25) (layer "B.Cu") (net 5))
 (segment (start 116.35 42.14) (end 112.02 42.14) (width 0.25) (layer "B.Cu") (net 5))
 (segment (start 122.361806 43.441806) (end 117.651806 43.441806) (width 0.25) (layer "B.Cu") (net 5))
 (segment (start 142.699981 42.47) (end 142.12 42.47) (width 0.25) (layer "B.Cu") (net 5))
 (segment (start 153.989194 37.88441) (end 154.541967 37.331637) (width 0.25) (layer "B.Cu") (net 5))
 (segment (start 120.07998 38.409701) (end 120.739519 41.408036) (width 0.25) (layer "B.Cu") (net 6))
 (segment (start 114.75 38.55) (end 116.91 36.39) (width 0.25) (layer "B.Cu") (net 3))
 (segment (start 116.91 36.39) (end 125.561377 36.39) (width 0.25) (layer "B.Cu") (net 3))
 (segment (start 125.561377 36.39) (end 127.751377 34.2) (width 0.25) (layer "B.Cu") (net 3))
 (segment (start 86.856115 52.917714) (end 89.083829 50.69) (width 0.25) (layer "B.Cu") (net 3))
 (segment (start 97.75 44.47) (end 100.68 44.47) (width 0.25) (layer "B.Cu") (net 3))
 (segment (start 154.041967 33.798014) (end 154.380571 33.45941) (width 0.25) (layer "B.Cu") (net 3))
 (segment (start 154.041967 34.88441) (end 154.041967 33.798014) (width 0.25) (layer "B.Cu") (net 3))
 (segment (start 161.816967 33.45941) (end 162.161967 33.80441) (width 0.25) (layer "B.Cu") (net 3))
 (segment (start 86.856115 54.922971) (end 86.856115 52.917714) (width 0.25) (layer "B.Cu") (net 3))
 (segment (start 153.802798 37.43441) (end 154.041967 37.195241) (width 0.25) (layer "B.Cu") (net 3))
 (segment (start 154.380571 33.45941) (end 161.816967 33.45941) (width 0.25) (layer "B.Cu") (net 3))
 (segment (start 154.041967 37.195241) (end 154.041967 34.88441) (width 0.25) (layer "B.Cu") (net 3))
 (segment (start 110.126367 38.55) (end 114.75 38.55) (width 0.25) (layer "B.Cu") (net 3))
 (segment (start 91.53 50.69) (end 97.75 44.47) (width 0.25) (layer "B.Cu") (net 3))
 (segment (start 143.132557 34.2) (end 146.366967 37.43441) (width 0.25) (layer "B.Cu") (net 3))
 (segment (start 146.366967 37.43441) (end 153.802798 37.43441) (width 0.25) (layer "B.Cu") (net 3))
 (segment (start 89.083829 50.69) (end 91.53 50.69) (width 0.25) (layer "B.Cu") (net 3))
 (segment (start 127.751377 34.2) (end 143.132557 34.2) (width 0.25) (layer "B.Cu") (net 3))
 (segment (start 104.755795 40.394205) (end 110.126367 38.55) (width 0.25) (layer "B.Cu") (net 3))
 (segment (start 100.68 44.47) (end 104.755795 40.394205) (width 0.25) (layer "B.Cu") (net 3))
 (segment (start 98.666105 47.058549) (end 100.263678 49.680144) (width 0.25) (layer "B.Cu") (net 4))
 (segment (start 156.041967 37.071979) (end 162.161967 43.191979) (width 0.25) (layer "B.Cu") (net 12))
 (segment (start 162.161967 43.191979) (end 162.161967 43.96441) (width 0.25) (layer "B.Cu") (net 12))
 (segment (start 156.041967 34.88441) (end 156.041967 37.071979) (width 0.25) (layer "B.Cu") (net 12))
 (segment (start 159.64485 41.700619) (end 159.921059 41.42441) (width 0.25) (layer "F.Cu") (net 13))
 (segment (start 159.921059 41.42441) (end 162.161967 41.42441) (width 0.25) (layer "F.Cu") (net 13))
 (via (at 159.64485 41.700619) (size 0.8) (drill 0.4) (layers "F.Cu" "B.Cu") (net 13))
 (segment (start 159.64485 41.700619) (end 159.64485 41.311258) (width 0.25) (layer "B.Cu") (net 13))
 (segment (start 159.64485 41.311258) (end 155.541967 37.208375) (width 0.25) (layer "B.Cu") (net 13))
 (segment (start 155.541967 37.208375) (end 155.541967 34.88441) (width 0.25) (layer "B.Cu") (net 13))
 (segment (start 153.541967 33.798014) (end 153.203363 33.45941) (width 0.25) (layer "B.Cu") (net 15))
 (segment (start 148.89941 33.45941) (end 146.921967 31.481967) (width 0.25) (layer "B.Cu") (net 15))
 (segment (start 153.541967 34.88441) (end 153.541967 33.798014) (width 0.25) (layer "B.Cu") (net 15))
 (segment (start 153.203363 33.45941) (end 148.89941 33.45941) (width 0.25) (layer "B.Cu") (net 15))
 (segment (start 146.921967 31.481967) (end 146.921967 31.26441) (width 0.25) (layer "B.Cu") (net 15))
 (segment (start 153.016967 33.90941) (end 149.75059 33.90941) (width 0.25) (layer "B.Cu") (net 16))
 (segment (start 149.75 33.91) (end 147.027557 33.91) (width 0.25) (layer "B.Cu") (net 16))
 (segment (start 153.041967 34.88441) (end 153.041967 33.93441) (width 0.25) (layer "B.Cu") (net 16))
 (segment (start 153.041967 33.93441) (end 153.016967 33.90941) (width 0.25) (layer "B.Cu") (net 16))
 (segment (start 147.027557 33.91) (end 146.921967 33.80441) (width 0.25) (layer "B.Cu") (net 16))
 (segment (start 149.75059 33.90941) (end 149.75 33.91) (width 0.25) (layer "B.Cu") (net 16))
 (segment (start 148.906377 34.36) (end 146.921967 36.34441) (width 0.25) (layer "B.Cu") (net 17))
 (segment (start 152.541967 34.88441) (end 152.016967 34.35941) (width 0.25) (layer "B.Cu") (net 17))
 (segment (start 149.936986 34.35941) (end 149.936396 34.36) (width 0.25) (layer "B.Cu") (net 17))
 (segment (start 149.936396 34.36) (end 148.906377 34.36) (width 0.25) (layer "B.Cu") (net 17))
 (segment (start 152.016967 34.35941) (end 149.936986 34.35941) (width 0.25) (layer "B.Cu") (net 17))
 (segment (start 147.226377 43.66) (end 153.35 43.66) (width 0.4) (layer "B.Cu") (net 1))
 (segment (start 162.89 37.62) (end 159.944557 37.62) (width 0.4) (layer "B.Cu") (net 1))
 (segment (start 152.741967 46.96441) (end 153.271967 46.43441) (width 0.25) (layer "B.Cu") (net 1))
 (segment (start 153.271967 46.43441) (end 153.271967 44.91741) (width 0.25) (layer "B.Cu") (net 1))
 (segment (start 153.271967 44.91741) (end 153.271967 43.738033) (width 0.25) (layer "B.Cu") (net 1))
 (segment (start 159.944557 37.62) (end 158.986967 36.66241) (width 0.4) (layer "B.Cu") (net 1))
 (segment (start 163.48 45.23) (end 163.48 38.21) (width 0.4) (layer "B.Cu") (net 1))
 (segment (start 146.921967 43.96441) (end 147.226377 43.66) (width 0.4) (layer "B.Cu") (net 1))
 (segment (start 156.341967 46.96441) (end 152.741967 46.96441) (width 0.25) (layer "B.Cu") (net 1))
 (segment (start 164.53441 46.28441) (end 163.48 45.23) (width 0.4) (layer "B.Cu") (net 1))
 (segment (start 159.78 43.66) (end 161.39 45.27) (width 0.4) (layer "B.Cu") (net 1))
 (segment (start 163.48 38.21) (end 162.89 37.62) (width 0.4) (layer "B.Cu") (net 1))
 (segment (start 175.791967 46.28441) (end 164.53441 46.28441) (width 0.4) (layer "B.Cu") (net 1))
 (segment (start 161.39 45.27) (end 163.35 45.27) (width 0.4) (layer "B.Cu") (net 1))
 (segment (start 153.35 43.66) (end 159.78 43.66) (width 0.4) (layer "B.Cu") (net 1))
 (segment (start 163.35 45.27) (end 163.48 45.14) (width 0.4) (layer "B.Cu") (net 1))
 (segment (start 153.271967 43.738033) (end 153.35 43.66) (width 0.25) (layer "B.Cu") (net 1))
 (segment (start 163.854734 45.19941) (end 163.839734 45.21441) (width 0.4) (layer "F.Cu") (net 9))
 (segment (start 163.839734 45.21441) (end 161.392033 45.21441) (width 0.4) (layer "F.Cu") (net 9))
 (segment (start 170.041967 46.34941) (end 168.891967 45.19941) (width 0.4) (layer "F.Cu") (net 9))
 (segment (start 157.86 39.694377) (end 158.986967 38.56741) (width 0.4) (layer "F.Cu") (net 9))
 (segment (start 157.86 41.682377) (end 157.86 39.694377) (width 0.4) (layer "F.Cu") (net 9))
 (segment (start 168.891967 45.19941) (end 163.854734 45.19941) (width 0.4) (layer "F.Cu") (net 9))
 (segment (start 161.392033 45.21441) (end 157.86 41.682377) (width 0.4) (layer "F.Cu") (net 9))
 (segment (start 156.18741 44.91741) (end 155.811967 44.91741) (width 0.25) (layer "B.Cu") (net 2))
 (segment (start 156.341967 48.40441) (end 157.291967 48.40441) (width 0.25) (layer "B.Cu") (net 2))
 (segment (start 157.291967 48.40441) (end 157.366967 48.32941) (width 0.25) (layer "B.Cu") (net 2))
 (segment (start 157.366967 46.096967) (end 156.18741 44.91741) (width 0.25) (layer "B.Cu") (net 2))
 (segment (start 157.366967 48.32941) (end 157.366967 46.096967) (width 0.25) (layer "B.Cu") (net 2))
 (segment (start 152.741967 48.40441) (end 156.341967 48.40441) (width 0.25) (layer "B.Cu") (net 2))
 (segment (start 175.791967 48.28441) (end 172.526967 48.28441) (width 0.4) (layer "F.Cu") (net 10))
 (segment (start 171.541967 47.29941) (end 171.541967 46.34941) (width 0.4) (layer "F.Cu") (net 10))
 (segment (start 172.526967 48.28441) (end 171.541967 47.29941) (width 0.4) (layer "F.Cu") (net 10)))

